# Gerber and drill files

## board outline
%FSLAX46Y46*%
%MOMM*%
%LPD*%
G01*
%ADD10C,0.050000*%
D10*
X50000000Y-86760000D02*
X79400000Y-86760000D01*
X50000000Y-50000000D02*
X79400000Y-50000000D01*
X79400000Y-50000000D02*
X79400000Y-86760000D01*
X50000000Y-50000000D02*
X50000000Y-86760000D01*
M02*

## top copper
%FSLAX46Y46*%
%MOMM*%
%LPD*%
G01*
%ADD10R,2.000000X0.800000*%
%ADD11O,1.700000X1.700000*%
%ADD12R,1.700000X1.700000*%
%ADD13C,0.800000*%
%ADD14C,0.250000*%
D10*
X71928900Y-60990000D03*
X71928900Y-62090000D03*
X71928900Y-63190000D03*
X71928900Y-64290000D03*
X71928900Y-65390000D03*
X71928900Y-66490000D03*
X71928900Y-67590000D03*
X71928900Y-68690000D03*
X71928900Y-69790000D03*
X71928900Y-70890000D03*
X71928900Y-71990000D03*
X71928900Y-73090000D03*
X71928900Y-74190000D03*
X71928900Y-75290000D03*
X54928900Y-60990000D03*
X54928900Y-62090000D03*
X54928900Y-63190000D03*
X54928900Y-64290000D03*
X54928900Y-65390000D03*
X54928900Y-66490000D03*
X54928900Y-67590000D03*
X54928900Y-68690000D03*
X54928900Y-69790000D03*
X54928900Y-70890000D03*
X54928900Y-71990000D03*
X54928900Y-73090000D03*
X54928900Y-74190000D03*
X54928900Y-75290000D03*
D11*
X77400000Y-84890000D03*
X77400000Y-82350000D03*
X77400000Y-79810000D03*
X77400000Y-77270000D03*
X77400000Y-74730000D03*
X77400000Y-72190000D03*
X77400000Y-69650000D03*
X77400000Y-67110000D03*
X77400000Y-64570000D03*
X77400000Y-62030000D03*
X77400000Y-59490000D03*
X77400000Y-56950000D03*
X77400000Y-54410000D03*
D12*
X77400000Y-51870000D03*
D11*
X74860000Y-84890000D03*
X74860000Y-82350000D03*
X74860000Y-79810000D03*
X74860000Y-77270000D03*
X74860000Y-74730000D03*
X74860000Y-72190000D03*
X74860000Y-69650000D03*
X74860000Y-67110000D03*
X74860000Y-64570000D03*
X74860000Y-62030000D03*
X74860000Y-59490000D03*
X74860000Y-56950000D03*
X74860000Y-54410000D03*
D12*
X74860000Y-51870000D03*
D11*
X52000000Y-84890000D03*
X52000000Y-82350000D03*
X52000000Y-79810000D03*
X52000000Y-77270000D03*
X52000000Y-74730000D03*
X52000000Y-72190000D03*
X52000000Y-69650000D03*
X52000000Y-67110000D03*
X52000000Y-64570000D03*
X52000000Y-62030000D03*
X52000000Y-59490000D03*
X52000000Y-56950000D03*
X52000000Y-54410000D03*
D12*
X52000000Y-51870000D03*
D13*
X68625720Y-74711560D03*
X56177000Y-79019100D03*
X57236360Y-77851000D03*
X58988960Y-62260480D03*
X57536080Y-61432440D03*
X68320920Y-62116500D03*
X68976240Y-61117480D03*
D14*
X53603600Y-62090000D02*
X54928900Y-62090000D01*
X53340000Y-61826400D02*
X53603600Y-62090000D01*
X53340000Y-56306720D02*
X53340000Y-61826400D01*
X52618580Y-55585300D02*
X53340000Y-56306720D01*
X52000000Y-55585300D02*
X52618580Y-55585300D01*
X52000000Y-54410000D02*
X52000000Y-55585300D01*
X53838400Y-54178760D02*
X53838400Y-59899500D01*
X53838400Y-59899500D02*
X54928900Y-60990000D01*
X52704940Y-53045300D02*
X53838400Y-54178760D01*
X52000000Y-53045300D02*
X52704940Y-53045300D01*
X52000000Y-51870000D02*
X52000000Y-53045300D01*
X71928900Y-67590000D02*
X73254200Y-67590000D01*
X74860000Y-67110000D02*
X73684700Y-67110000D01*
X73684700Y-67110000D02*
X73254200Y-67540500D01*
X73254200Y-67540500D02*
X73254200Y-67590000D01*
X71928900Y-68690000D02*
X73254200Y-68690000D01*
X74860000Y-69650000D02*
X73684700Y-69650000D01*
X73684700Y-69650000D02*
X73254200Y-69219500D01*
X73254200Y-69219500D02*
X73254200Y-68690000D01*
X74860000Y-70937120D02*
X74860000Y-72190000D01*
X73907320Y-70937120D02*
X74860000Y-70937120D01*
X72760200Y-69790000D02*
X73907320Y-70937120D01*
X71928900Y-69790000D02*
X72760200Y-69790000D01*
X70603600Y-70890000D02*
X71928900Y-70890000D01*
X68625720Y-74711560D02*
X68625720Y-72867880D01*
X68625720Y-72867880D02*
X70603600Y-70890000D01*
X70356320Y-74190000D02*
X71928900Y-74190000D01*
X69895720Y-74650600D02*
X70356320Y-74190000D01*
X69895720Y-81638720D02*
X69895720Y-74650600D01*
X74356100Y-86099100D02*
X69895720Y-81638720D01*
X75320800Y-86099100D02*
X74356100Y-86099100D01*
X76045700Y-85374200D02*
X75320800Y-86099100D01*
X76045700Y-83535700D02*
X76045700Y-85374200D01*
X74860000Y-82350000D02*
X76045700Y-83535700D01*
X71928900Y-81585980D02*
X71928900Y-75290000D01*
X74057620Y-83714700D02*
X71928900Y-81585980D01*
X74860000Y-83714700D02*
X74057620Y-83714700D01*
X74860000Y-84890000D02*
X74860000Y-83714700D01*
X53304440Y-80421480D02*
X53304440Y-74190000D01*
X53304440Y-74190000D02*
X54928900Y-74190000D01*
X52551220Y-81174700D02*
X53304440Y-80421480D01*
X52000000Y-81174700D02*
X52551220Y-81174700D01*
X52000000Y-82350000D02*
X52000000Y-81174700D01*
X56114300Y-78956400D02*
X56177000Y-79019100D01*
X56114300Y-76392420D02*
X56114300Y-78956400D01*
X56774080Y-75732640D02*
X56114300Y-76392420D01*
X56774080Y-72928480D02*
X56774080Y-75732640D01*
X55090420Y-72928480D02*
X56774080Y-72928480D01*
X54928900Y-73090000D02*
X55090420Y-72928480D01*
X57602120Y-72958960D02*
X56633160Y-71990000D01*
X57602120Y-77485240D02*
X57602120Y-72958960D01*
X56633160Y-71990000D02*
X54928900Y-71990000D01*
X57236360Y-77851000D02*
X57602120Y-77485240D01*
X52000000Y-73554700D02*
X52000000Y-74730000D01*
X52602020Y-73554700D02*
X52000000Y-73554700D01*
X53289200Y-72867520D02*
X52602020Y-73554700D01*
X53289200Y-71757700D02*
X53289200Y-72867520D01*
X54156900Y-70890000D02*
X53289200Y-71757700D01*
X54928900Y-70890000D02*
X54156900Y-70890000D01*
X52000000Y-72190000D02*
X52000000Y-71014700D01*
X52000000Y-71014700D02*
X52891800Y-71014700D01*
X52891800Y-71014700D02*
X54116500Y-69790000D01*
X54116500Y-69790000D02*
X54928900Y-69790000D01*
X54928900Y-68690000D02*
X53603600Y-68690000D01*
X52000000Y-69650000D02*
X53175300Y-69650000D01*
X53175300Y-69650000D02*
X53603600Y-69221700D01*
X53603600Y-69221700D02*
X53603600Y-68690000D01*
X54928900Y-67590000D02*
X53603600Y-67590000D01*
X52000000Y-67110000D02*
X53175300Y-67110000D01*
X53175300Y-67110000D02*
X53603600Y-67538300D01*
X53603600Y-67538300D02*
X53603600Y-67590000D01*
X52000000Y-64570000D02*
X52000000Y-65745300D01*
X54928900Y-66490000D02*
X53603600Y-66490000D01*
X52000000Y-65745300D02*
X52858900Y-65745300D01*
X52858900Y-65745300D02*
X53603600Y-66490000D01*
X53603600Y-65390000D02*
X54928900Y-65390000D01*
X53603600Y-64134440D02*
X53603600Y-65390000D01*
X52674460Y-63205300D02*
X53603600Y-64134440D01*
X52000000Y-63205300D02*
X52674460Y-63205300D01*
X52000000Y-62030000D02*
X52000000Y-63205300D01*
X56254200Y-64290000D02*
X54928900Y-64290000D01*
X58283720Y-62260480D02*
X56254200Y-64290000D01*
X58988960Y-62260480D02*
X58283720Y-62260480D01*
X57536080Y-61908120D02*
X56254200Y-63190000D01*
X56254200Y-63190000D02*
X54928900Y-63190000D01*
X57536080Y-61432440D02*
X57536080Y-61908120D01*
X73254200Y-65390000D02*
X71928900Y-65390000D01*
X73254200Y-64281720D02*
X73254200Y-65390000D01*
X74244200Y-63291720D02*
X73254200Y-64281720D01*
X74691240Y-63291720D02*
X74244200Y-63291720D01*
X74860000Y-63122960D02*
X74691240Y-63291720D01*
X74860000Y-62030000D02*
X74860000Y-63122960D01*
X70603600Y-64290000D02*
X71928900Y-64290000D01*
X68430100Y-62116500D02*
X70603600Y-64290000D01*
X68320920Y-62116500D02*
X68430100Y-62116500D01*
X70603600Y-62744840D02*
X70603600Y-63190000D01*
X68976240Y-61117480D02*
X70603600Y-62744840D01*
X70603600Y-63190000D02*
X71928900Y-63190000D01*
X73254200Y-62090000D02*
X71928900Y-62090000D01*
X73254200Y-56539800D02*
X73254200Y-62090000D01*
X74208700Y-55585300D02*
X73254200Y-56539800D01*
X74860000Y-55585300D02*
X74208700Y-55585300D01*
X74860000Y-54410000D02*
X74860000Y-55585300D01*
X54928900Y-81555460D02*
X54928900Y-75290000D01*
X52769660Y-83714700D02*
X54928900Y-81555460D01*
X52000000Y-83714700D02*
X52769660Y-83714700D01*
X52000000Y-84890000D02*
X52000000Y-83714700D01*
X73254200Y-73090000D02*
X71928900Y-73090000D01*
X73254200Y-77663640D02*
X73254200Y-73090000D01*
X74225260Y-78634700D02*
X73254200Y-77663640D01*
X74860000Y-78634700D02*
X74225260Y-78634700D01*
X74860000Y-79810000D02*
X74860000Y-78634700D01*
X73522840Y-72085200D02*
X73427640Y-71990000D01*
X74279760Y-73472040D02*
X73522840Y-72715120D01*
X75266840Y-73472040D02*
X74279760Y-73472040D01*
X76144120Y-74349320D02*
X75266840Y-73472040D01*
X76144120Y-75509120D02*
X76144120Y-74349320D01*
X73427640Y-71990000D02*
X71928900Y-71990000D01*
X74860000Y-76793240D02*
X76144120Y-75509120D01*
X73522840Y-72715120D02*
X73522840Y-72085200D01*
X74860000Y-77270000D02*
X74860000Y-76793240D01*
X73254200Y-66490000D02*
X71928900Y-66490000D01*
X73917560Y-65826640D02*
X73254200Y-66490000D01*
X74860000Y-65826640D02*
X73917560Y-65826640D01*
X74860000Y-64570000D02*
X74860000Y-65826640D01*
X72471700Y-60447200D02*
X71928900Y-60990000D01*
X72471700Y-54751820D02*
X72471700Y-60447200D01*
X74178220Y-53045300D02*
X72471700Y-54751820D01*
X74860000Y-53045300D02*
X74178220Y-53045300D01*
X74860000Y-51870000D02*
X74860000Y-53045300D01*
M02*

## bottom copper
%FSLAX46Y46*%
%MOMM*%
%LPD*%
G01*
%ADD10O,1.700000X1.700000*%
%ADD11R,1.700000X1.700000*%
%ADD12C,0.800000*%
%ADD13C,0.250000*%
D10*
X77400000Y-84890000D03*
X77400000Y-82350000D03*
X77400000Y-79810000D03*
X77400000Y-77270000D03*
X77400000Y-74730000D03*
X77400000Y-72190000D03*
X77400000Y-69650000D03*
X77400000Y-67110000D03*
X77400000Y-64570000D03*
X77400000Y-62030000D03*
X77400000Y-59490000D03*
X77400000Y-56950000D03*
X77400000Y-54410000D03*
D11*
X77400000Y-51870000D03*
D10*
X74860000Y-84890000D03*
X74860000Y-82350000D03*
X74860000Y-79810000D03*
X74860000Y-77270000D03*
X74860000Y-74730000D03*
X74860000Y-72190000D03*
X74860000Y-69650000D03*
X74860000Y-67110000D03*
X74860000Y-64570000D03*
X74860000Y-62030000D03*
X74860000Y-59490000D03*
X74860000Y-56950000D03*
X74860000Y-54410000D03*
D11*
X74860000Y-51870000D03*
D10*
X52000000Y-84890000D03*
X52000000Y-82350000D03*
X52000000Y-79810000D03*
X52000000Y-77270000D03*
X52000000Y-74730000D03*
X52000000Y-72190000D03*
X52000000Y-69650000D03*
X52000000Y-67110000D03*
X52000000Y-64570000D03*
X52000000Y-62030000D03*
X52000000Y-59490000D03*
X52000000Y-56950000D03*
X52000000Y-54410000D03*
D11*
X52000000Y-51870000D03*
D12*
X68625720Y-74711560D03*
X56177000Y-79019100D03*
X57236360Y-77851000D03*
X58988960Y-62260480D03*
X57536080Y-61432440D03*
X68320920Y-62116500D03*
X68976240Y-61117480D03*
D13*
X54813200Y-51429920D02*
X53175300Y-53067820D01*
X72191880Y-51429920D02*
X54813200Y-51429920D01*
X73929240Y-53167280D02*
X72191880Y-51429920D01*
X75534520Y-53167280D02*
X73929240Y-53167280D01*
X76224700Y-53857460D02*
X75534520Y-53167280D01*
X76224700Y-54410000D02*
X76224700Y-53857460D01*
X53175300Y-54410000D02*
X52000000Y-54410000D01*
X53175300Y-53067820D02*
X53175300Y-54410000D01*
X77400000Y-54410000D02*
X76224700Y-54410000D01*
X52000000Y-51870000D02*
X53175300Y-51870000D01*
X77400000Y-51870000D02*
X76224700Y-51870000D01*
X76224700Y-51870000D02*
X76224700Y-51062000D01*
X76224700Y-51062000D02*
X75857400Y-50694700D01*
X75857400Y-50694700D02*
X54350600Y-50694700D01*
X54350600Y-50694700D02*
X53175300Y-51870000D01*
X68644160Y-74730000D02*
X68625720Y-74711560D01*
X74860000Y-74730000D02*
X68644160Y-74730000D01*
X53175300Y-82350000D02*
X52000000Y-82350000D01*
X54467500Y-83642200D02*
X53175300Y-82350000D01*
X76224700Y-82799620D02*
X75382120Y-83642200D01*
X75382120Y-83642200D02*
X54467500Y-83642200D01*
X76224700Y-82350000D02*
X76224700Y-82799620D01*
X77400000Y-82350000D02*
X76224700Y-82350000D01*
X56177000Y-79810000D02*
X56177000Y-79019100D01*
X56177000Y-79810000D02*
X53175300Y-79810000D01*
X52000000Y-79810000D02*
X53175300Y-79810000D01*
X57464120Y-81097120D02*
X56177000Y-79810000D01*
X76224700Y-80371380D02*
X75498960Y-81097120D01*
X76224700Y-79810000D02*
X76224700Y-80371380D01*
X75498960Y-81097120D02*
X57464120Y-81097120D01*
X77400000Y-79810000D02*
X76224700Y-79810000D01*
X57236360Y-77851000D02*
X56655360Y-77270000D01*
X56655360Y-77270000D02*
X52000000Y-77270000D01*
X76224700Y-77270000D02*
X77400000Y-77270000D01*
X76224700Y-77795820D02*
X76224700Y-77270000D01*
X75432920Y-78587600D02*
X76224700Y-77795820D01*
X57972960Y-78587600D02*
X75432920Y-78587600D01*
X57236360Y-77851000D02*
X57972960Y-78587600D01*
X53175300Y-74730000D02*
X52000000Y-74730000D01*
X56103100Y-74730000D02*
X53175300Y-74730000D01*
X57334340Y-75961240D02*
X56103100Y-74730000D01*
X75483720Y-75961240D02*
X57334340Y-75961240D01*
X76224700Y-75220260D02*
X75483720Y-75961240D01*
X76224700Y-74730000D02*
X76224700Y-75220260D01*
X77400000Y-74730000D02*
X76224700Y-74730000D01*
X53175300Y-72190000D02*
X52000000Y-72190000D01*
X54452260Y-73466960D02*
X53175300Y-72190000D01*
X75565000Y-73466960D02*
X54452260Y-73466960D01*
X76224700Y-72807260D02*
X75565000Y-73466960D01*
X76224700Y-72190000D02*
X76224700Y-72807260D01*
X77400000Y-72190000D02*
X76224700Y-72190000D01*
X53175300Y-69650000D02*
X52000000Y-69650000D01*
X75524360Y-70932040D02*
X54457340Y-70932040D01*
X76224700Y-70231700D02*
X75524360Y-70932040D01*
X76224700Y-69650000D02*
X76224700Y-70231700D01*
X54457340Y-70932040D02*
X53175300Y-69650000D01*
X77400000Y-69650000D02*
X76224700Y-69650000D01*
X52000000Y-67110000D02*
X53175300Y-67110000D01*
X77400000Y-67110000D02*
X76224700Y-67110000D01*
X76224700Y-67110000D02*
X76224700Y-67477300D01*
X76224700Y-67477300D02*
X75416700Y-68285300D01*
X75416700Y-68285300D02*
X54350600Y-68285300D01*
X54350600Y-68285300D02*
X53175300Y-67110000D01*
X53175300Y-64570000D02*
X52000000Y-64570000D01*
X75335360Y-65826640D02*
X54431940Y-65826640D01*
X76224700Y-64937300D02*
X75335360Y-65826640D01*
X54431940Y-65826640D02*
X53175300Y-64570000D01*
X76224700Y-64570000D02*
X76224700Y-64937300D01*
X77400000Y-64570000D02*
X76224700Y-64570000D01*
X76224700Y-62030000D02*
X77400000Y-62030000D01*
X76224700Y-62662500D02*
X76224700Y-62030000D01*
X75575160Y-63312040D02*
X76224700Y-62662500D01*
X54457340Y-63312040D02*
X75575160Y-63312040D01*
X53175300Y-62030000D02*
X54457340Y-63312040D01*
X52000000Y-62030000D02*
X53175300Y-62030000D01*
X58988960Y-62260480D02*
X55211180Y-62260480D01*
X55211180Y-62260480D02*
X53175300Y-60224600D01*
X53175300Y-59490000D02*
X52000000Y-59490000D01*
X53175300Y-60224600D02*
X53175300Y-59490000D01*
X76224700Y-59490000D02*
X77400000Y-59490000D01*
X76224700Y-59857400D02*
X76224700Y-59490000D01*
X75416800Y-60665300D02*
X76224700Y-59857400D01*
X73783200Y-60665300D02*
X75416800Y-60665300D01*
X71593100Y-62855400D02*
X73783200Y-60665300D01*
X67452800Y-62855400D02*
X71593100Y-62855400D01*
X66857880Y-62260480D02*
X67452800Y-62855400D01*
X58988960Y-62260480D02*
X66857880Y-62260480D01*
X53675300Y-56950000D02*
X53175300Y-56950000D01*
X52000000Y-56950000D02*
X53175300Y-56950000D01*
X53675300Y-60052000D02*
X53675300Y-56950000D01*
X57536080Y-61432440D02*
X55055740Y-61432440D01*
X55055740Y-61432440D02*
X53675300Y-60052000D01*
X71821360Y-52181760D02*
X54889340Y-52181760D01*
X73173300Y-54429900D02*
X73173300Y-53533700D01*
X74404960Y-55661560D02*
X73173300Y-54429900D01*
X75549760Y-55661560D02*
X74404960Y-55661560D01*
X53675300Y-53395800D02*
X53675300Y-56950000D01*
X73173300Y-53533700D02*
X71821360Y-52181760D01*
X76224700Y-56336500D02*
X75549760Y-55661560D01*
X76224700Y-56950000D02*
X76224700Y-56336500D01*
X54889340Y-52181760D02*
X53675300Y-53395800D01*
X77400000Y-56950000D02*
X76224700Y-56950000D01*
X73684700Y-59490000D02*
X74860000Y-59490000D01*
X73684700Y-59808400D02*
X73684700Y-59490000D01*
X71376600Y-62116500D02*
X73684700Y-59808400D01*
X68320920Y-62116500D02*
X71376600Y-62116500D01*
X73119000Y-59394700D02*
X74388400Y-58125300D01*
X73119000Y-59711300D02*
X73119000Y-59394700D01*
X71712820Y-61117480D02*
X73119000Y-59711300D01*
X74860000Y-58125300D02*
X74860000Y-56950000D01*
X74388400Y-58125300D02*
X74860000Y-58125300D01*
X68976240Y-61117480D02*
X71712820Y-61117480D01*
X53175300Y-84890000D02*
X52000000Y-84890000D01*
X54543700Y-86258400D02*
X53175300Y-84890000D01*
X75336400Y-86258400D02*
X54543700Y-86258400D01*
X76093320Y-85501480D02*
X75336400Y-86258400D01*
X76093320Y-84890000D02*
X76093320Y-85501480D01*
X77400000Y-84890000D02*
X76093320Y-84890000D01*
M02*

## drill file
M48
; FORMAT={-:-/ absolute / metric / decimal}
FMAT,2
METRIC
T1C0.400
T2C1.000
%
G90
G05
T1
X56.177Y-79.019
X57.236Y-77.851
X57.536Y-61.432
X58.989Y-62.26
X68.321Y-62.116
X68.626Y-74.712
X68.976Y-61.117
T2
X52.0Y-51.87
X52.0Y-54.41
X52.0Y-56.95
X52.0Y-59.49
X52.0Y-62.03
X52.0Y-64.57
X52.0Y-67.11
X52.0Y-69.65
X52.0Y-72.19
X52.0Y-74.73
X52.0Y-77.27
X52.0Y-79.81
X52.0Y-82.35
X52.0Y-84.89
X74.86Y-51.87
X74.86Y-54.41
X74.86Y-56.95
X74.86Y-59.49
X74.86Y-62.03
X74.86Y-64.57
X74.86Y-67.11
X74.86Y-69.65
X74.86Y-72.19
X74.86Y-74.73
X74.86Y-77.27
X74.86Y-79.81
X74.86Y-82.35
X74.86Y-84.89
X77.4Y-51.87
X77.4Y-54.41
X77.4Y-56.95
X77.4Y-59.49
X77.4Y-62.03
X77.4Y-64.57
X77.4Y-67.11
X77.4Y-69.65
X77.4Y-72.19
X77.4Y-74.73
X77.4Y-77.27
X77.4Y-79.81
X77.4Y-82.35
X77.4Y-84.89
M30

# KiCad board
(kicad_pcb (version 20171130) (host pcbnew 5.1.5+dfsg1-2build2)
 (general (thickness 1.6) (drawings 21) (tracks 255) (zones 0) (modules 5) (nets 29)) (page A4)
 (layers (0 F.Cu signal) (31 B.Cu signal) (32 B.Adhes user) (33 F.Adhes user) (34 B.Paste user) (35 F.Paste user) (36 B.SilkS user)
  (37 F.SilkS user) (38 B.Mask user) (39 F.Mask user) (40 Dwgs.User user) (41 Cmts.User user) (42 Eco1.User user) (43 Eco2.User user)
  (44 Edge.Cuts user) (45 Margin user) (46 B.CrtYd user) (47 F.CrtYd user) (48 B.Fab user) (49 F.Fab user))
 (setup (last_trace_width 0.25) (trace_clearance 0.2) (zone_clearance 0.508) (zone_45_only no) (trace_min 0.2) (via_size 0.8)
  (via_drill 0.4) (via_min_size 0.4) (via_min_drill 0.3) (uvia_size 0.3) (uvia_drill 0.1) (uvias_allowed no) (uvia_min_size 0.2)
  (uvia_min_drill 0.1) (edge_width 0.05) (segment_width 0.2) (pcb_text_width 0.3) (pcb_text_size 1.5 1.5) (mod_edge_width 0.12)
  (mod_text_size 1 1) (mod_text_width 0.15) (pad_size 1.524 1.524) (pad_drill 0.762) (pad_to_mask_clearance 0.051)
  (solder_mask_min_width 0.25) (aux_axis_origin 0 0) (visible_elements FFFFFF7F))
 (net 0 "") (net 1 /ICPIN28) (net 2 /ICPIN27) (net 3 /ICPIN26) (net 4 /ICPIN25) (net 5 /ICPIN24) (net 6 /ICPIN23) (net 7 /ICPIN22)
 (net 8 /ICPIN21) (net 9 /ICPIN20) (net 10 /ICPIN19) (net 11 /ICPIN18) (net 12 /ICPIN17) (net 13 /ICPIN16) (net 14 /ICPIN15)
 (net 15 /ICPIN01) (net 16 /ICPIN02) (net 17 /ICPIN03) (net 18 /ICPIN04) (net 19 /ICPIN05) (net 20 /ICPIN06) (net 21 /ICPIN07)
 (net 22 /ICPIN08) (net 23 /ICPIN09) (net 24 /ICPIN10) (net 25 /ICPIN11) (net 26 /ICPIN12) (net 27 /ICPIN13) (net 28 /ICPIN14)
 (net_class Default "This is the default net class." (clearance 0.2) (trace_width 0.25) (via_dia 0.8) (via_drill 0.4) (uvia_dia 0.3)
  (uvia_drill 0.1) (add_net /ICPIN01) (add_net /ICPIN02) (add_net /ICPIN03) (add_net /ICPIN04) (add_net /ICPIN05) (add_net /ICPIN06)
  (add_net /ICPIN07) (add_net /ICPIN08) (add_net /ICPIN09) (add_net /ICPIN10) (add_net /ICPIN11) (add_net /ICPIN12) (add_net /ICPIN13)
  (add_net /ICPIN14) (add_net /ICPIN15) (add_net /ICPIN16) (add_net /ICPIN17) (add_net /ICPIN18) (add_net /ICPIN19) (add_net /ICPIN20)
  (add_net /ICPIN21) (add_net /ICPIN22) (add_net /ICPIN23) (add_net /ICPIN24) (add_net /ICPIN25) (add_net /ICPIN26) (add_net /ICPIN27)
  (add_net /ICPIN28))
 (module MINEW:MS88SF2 (layer F.Cu) (at 63.4289 65)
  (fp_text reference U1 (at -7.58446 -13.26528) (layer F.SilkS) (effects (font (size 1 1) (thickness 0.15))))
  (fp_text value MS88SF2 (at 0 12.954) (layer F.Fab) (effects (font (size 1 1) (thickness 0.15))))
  (pad 28 smd rect (at 8.5 -4.01) (size 2 0.8) (layers F.Cu F.Paste F.Mask) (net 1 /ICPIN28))
  (pad 27 smd rect (at 8.5 -2.91) (size 2 0.8) (layers F.Cu F.Paste F.Mask) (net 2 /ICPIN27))
  (pad 26 smd rect (at 8.5 -1.81) (size 2 0.8) (layers F.Cu F.Paste F.Mask) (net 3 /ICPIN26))
  (pad 25 smd rect (at 8.5 -0.71) (size 2 0.8) (layers F.Cu F.Paste F.Mask) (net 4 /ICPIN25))
  (pad 24 smd rect (at 8.5 0.39) (size 2 0.8) (layers F.Cu F.Paste F.Mask) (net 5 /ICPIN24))
  (pad 23 smd rect (at 8.5 1.49) (size 2 0.8) (layers F.Cu F.Paste F.Mask) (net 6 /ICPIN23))
  (pad 22 smd rect (at 8.5 2.59) (size 2 0.8) (layers F.Cu F.Paste F.Mask) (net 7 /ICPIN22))
  (pad 21 smd rect (at 8.5 3.69) (size 2 0.8) (layers F.Cu F.Paste F.Mask) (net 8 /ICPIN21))
  (pad 20 smd rect (at 8.5 4.79) (size 2 0.8) (layers F.Cu F.Paste F.Mask) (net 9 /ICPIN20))
  (pad 19 smd rect (at 8.5 5.89) (size 2 0.8) (layers F.Cu F.Paste F.Mask) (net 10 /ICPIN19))
  (pad 18 smd rect (at 8.5 6.99) (size 2 0.8) (layers F.Cu F.Paste F.Mask) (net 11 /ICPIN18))
  (pad 17 smd rect (at 8.5 8.09) (size 2 0.8) (layers F.Cu F.Paste F.Mask) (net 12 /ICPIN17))
  (pad 16 smd rect (at 8.5 9.19) (size 2 0.8) (layers F.Cu F.Paste F.Mask) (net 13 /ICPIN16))
  (pad 15 smd rect (at 8.5 10.29) (size 2 0.8) (layers F.Cu F.Paste F.Mask) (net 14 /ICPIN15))
  (pad 1 smd rect (at -8.5 -4.01) (size 2 0.8) (layers F.Cu F.Paste F.Mask) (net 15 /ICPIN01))
  (pad 2 smd rect (at -8.5 -2.91) (size 2 0.8) (layers F.Cu F.Paste F.Mask) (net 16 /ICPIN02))
  (pad 3 smd rect (at -8.5 -1.81) (size 2 0.8) (layers F.Cu F.Paste F.Mask) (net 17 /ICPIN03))
  (pad 4 smd rect (at -8.5 -0.71) (size 2 0.8) (layers F.Cu F.Paste F.Mask) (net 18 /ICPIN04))
  (pad 5 smd rect (at -8.5 0.39) (size 2 0.8) (layers F.Cu F.Paste F.Mask) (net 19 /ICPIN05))
  (pad 6 smd rect (at -8.5 1.49) (size 2 0.8) (layers F.Cu F.Paste F.Mask) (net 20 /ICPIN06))
  (pad 7 smd rect (at -8.5 2.59) (size 2 0.8) (layers F.Cu F.Paste F.Mask) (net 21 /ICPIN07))
  (pad 8 smd rect (at -8.5 3.69) (size 2 0.8) (layers F.Cu F.Paste F.Mask) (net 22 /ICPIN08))
  (pad 9 smd rect (at -8.5 4.79) (size 2 0.8) (layers F.Cu F.Paste F.Mask) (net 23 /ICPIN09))
  (pad 10 smd rect (at -8.5 5.89) (size 2 0.8) (layers F.Cu F.Paste F.Mask) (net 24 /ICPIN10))
  (pad 11 smd rect (at -8.5 6.99) (size 2 0.8) (layers F.Cu F.Paste F.Mask) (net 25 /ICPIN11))
  (pad 12 smd rect (at -8.5 8.09) (size 2 0.8) (layers F.Cu F.Paste F.Mask) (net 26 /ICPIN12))
  (pad 13 smd rect (at -8.5 9.19) (size 2 0.8) (layers F.Cu F.Paste F.Mask) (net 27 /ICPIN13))
  (pad 14 smd rect (at -8.5 10.29) (size 2 0.8) (layers F.Cu F.Paste F.Mask) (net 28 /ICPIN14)))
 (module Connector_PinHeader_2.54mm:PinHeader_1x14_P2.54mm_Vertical (layer F.Cu) (at 77.4 51.87)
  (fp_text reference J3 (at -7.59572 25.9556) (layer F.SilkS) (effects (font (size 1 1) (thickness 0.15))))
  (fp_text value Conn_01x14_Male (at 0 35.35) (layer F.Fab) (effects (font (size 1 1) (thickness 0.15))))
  (pad 14 thru_hole oval (at 0 33.02) (size 1.7 1.7) (drill 1) (layers *.Cu *.Mask) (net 28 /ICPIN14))
  (pad 13 thru_hole oval (at 0 30.48) (size 1.7 1.7) (drill 1) (layers *.Cu *.Mask) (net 27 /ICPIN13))
  (pad 12 thru_hole oval (at 0 27.94) (size 1.7 1.7) (drill 1) (layers *.Cu *.Mask) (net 26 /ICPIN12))
  (pad 11 thru_hole oval (at 0 25.4) (size 1.7 1.7) (drill 1) (layers *.Cu *.Mask) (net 25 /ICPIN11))
  (pad 10 thru_hole oval (at 0 22.86) (size 1.7 1.7) (drill 1) (layers *.Cu *.Mask) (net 24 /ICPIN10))
  (pad 9 thru_hole oval (at 0 20.32) (size 1.7 1.7) (drill 1) (layers *.Cu *.Mask) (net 23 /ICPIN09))
  (pad 8 thru_hole oval (at 0 17.78) (size 1.7 1.7) (drill 1) (layers *.Cu *.Mask) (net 22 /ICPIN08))
  (pad 7 thru_hole oval (at 0 15.24) (size 1.7 1.7) (drill 1) (layers *.Cu *.Mask) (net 21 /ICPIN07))
  (pad 6 thru_hole oval (at 0 12.7) (size 1.7 1.7) (drill 1) (layers *.Cu *.Mask) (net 20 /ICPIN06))
  (pad 5 thru_hole oval (at 0 10.16) (size 1.7 1.7) (drill 1) (layers *.Cu *.Mask) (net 19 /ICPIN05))
  (pad 4 thru_hole oval (at 0 7.62) (size 1.7 1.7) (drill 1) (layers *.Cu *.Mask) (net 18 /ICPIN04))
  (pad 3 thru_hole oval (at 0 5.08) (size 1.7 1.7) (drill 1) (layers *.Cu *.Mask) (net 17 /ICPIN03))
  (pad 2 thru_hole oval (at 0 2.54) (size 1.7 1.7) (drill 1) (layers *.Cu *.Mask) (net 16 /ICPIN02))
  (pad 1 thru_hole rect (at 0 0) (size 1.7 1.7) (drill 1) (layers *.Cu *.Mask) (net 15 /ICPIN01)))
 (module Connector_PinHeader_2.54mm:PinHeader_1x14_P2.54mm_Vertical (layer F.Cu) (at 74.86 51.87)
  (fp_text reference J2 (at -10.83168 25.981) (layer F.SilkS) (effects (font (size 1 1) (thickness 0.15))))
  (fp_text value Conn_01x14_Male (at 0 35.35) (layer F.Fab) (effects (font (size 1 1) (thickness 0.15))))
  (pad 14 thru_hole oval (at 0 33.02) (size 1.7 1.7) (drill 1) (layers *.Cu *.Mask) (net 14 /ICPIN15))
  (pad 13 thru_hole oval (at 0 30.48) (size 1.7 1.7) (drill 1) (layers *.Cu *.Mask) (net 13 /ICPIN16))
  (pad 12 thru_hole oval (at 0 27.94) (size 1.7 1.7) (drill 1) (layers *.Cu *.Mask) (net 12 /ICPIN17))
  (pad 11 thru_hole oval (at 0 25.4) (size 1.7 1.7) (drill 1) (layers *.Cu *.Mask) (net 11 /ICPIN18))
  (pad 10 thru_hole oval (at 0 22.86) (size 1.7 1.7) (drill 1) (layers *.Cu *.Mask) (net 10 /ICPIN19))
  (pad 9 thru_hole oval (at 0 20.32) (size 1.7 1.7) (drill 1) (layers *.Cu *.Mask) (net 9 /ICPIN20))
  (pad 8 thru_hole oval (at 0 17.78) (size 1.7 1.7) (drill 1) (layers *.Cu *.Mask) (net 8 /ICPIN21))
  (pad 7 thru_hole oval (at 0 15.24) (size 1.7 1.7) (drill 1) (layers *.Cu *.Mask) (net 7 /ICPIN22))
  (pad 6 thru_hole oval (at 0 12.7) (size 1.7 1.7) (drill 1) (layers *.Cu *.Mask) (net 6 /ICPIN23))
  (pad 5 thru_hole oval (at 0 10.16) (size 1.7 1.7) (drill 1) (layers *.Cu *.Mask) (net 5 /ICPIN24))
  (pad 4 thru_hole oval (at 0 7.62) (size 1.7 1.7) (drill 1) (layers *.Cu *.Mask) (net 4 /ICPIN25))
  (pad 3 thru_hole oval (at 0 5.08) (size 1.7 1.7) (drill 1) (layers *.Cu *.Mask) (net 3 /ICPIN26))
  (pad 2 thru_hole oval (at 0 2.54) (size 1.7 1.7) (drill 1) (layers *.Cu *.Mask) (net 2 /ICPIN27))
  (pad 1 thru_hole rect (at 0 0) (size 1.7 1.7) (drill 1) (layers *.Cu *.Mask) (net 1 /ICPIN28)))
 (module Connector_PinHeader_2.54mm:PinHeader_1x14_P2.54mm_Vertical (layer F.Cu) (at 52 51.87)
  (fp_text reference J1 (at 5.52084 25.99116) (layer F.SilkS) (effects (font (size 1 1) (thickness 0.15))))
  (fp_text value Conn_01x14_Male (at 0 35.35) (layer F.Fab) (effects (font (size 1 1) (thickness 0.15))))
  (pad 14 thru_hole oval (at 0 33.02) (size 1.7 1.7) (drill 1) (layers *.Cu *.Mask) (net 28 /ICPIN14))
  (pad 13 thru_hole oval (at 0 30.48) (size 1.7 1.7) (drill 1) (layers *.Cu *.Mask) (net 27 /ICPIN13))
  (pad 12 thru_hole oval (at 0 27.94) (size 1.7 1.7) (drill 1) (layers *.Cu *.Mask) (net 26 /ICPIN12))
  (pad 11 thru_hole oval (at 0 25.4) (size 1.7 1.7) (drill 1) (layers *.Cu *.Mask) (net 25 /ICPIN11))
  (pad 10 thru_hole oval (at 0 22.86) (size 1.7 1.7) (drill 1) (layers *.Cu *.Mask) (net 24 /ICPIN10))
  (pad 9 thru_hole oval (at 0 20.32) (size 1.7 1.7) (drill 1) (layers *.Cu *.Mask) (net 23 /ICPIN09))
  (pad 8 thru_hole oval (at 0 17.78) (size 1.7 1.7) (drill 1) (layers *.Cu *.Mask) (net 22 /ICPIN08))
  (pad 7 thru_hole oval (at 0 15.24) (size 1.7 1.7) (drill 1) (layers *.Cu *.Mask) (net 21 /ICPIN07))
  (pad 6 thru_hole oval (at 0 12.7) (size 1.7 1.7) (drill 1) (layers *.Cu *.Mask) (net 20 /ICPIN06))
  (pad 5 thru_hole oval (at 0 10.16) (size 1.7 1.7) (drill 1) (layers *.Cu *.Mask) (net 19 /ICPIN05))
  (pad 4 thru_hole oval (at 0 7.62) (size 1.7 1.7) (drill 1) (layers *.Cu *.Mask) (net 18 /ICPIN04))
  (pad 3 thru_hole oval (at 0 5.08) (size 1.7 1.7) (drill 1) (layers *.Cu *.Mask) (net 17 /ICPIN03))
  (pad 2 thru_hole oval (at 0 2.54) (size 1.7 1.7) (drill 1) (layers *.Cu *.Mask) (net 16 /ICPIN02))
  (pad 1 thru_hole rect (at 0 0) (size 1.7 1.7) (drill 1) (layers *.Cu *.Mask) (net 15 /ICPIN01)))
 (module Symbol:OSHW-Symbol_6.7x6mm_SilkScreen (layer F.Cu) (at 63.2714 56.68264)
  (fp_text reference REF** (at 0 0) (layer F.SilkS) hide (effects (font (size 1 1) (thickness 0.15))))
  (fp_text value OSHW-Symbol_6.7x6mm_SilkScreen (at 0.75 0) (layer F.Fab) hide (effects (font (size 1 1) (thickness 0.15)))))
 (gr_line (start 50 86.76) (end 79.4 86.76) (layer Edge.Cuts) (width 0.05))
 (gr_line (start 50 50) (end 79.4 50) (layer Edge.Cuts) (width 0.05))
 (gr_line (start 79.4 50) (end 79.4 86.76) (layer Edge.Cuts) (width 0.05))
 (gr_line (start 50 50) (end 50 86.76) (layer Edge.Cuts) (width 0.05))
 (segment (start 54.8132 51.42992) (end 53.1753 53.06782) (width 0.25) (layer B.Cu) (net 16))
 (segment (start 72.19188 51.42992) (end 54.8132 51.42992) (width 0.25) (layer B.Cu) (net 16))
 (segment (start 73.92924 53.16728) (end 72.19188 51.42992) (width 0.25) (layer B.Cu) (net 16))
 (segment (start 75.53452 53.16728) (end 73.92924 53.16728) (width 0.25) (layer B.Cu) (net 16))
 (segment (start 76.2247 53.85746) (end 75.53452 53.16728) (width 0.25) (layer B.Cu) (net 16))
 (segment (start 76.2247 54.41) (end 76.2247 53.85746) (width 0.25) (layer B.Cu) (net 16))
 (segment (start 53.1753 54.41) (end 52 54.41) (width 0.25) (layer B.Cu) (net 16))
 (segment (start 53.1753 53.06782) (end 53.1753 54.41) (width 0.25) (layer B.Cu) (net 16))
 (segment (start 77.4 54.41) (end 76.2247 54.41) (width 0.25) (layer B.Cu) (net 16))
 (segment (start 53.6036 62.09) (end 54.9289 62.09) (width 0.25) (layer F.Cu) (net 16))
 (segment (start 53.34 61.8264) (end 53.6036 62.09) (width 0.25) (layer F.Cu) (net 16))
 (segment (start 53.34 56.30672) (end 53.34 61.8264) (width 0.25) (layer F.Cu) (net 16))
 (segment (start 52.61858 55.5853) (end 53.34 56.30672) (width 0.25) (layer F.Cu) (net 16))
 (segment (start 52 55.5853) (end 52.61858 55.5853) (width 0.25) (layer F.Cu) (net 16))
 (segment (start 52 54.41) (end 52 55.5853) (width 0.25) (layer F.Cu) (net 16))
 (segment (start 52 51.87) (end 53.1753 51.87) (width 0.25) (layer B.Cu) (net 15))
 (segment (start 77.4 51.87) (end 76.2247 51.87) (width 0.25) (layer B.Cu) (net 15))
 (segment (start 76.2247 51.87) (end 76.2247 51.062) (width 0.25) (layer B.Cu) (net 15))
 (segment (start 76.2247 51.062) (end 75.8574 50.6947) (width 0.25) (layer B.Cu) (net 15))
 (segment (start 75.8574 50.6947) (end 54.3506 50.6947) (width 0.25) (layer B.Cu) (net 15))
 (segment (start 54.3506 50.6947) (end 53.1753 51.87) (width 0.25) (layer B.Cu) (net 15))
 (segment (start 53.8384 54.17876) (end 53.8384 59.8995) (width 0.25) (layer F.Cu) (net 15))
 (segment (start 53.8384 59.8995) (end 54.9289 60.99) (width 0.25) (layer F.Cu) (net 15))
 (segment (start 52.70494 53.0453) (end 53.8384 54.17876) (width 0.25) (layer F.Cu) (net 15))
 (segment (start 52 53.0453) (end 52.70494 53.0453) (width 0.25) (layer F.Cu) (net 15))
 (segment (start 52 51.87) (end 52 53.0453) (width 0.25) (layer F.Cu) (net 15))
 (segment (start 71.9289 67.59) (end 73.2542 67.59) (width 0.25) (layer F.Cu) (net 7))
 (segment (start 74.86 67.11) (end 73.6847 67.11) (width 0.25) (layer F.Cu) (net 7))
 (segment (start 73.6847 67.11) (end 73.2542 67.5405) (width 0.25) (layer F.Cu) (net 7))
 (segment (start 73.2542 67.5405) (end 73.2542 67.59) (width 0.25) (layer F.Cu) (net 7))
 (segment (start 71.9289 68.69) (end 73.2542 68.69) (width 0.25) (layer F.Cu) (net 8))
 (segment (start 74.86 69.65) (end 73.6847 69.65) (width 0.25) (layer F.Cu) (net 8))
 (segment (start 73.6847 69.65) (end 73.2542 69.2195) (width 0.25) (layer F.Cu) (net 8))
 (segment (start 73.2542 69.2195) (end 73.2542 68.69) (width 0.25) (layer F.Cu) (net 8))
 (segment (start 74.86 70.93712) (end 74.86 72.19) (width 0.25) (layer F.Cu) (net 9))
 (segment (start 73.90732 70.93712) (end 74.86 70.93712) (width 0.25) (layer F.Cu) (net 9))
 (segment (start 72.7602 69.79) (end 73.90732 70.93712) (width 0.25) (layer F.Cu) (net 9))
 (segment (start 71.9289 69.79) (end 72.7602 69.79) (width 0.25) (layer F.Cu) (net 9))
 (segment (start 70.6036 70.89) (end 71.9289 70.89) (width 0.25) (layer F.Cu) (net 10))
 (segment (start 68.62572 74.71156) (end 68.62572 72.86788) (width 0.25) (layer F.Cu) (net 10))
 (segment (start 68.64416 74.73) (end 68.62572 74.71156) (width 0.25) (layer B.Cu) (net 10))
 (segment (start 68.62572 72.86788) (end 70.6036 70.89) (width 0.25) (layer F.Cu) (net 10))
 (segment (start 74.86 74.73) (end 68.64416 74.73) (width 0.25) (layer B.Cu) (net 10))
 (via (at 68.62572 74.71156) (size 0.8) (drill 0.4) (layers F.Cu B.Cu) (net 10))
 (segment (start 70.35632 74.19) (end 71.9289 74.19) (width 0.25) (layer F.Cu) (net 13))
 (segment (start 69.89572 74.6506) (end 70.35632 74.19) (width 0.25) (layer F.Cu) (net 13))
 (segment (start 69.89572 81.63872) (end 69.89572 74.6506) (width 0.25) (layer F.Cu) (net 13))
 (segment (start 74.3561 86.0991) (end 69.89572 81.63872) (width 0.25) (layer F.Cu) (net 13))
 (segment (start 75.3208 86.0991) (end 74.3561 86.0991) (width 0.25) (layer F.Cu) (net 13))
 (segment (start 76.0457 85.3742) (end 75.3208 86.0991) (width 0.25) (layer F.Cu) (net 13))
 (segment (start 76.0457 83.5357) (end 76.0457 85.3742) (width 0.25) (layer F.Cu) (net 13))
 (segment (start 74.86 82.35) (end 76.0457 83.5357) (width 0.25) (layer F.Cu) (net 13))
 (segment (start 71.9289 81.58598) (end 71.9289 75.29) (width 0.25) (layer F.Cu) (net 14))
 (segment (start 74.05762 83.7147) (end 71.9289 81.58598) (width 0.25) (layer F.Cu) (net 14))
 (segment (start 74.86 83.7147) (end 74.05762 83.7147) (width 0.25) (layer F.Cu) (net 14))
 (segment (start 74.86 84.89) (end 74.86 83.7147) (width 0.25) (layer F.Cu) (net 14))
 (segment (start 53.1753 82.35) (end 52 82.35) (width 0.25) (layer B.Cu) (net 27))
 (segment (start 54.4675 83.6422) (end 53.1753 82.35) (width 0.25) (layer B.Cu) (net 27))
 (segment (start 76.2247 82.79962) (end 75.38212 83.6422) (width 0.25) (layer B.Cu) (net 27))
 (segment (start 75.38212 83.6422) (end 54.4675 83.6422) (width 0.25) (layer B.Cu) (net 27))
 (segment (start 76.2247 82.35) (end 76.2247 82.79962) (width 0.25) (layer B.Cu) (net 27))
 (segment (start 77.4 82.35) (end 76.2247 82.35) (width 0.25) (layer B.Cu) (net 27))
 (segment (start 53.30444 80.42148) (end 53.30444 74.19) (width 0.25) (layer F.Cu) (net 27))
 (segment (start 53.30444 74.19) (end 54.9289 74.19) (width 0.25) (layer F.Cu) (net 27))
 (segment (start 52.55122 81.1747) (end 53.30444 80.42148) (width 0.25) (layer F.Cu) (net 27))
 (segment (start 52 81.1747) (end 52.55122 81.1747) (width 0.25) (layer F.Cu) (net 27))
 (segment (start 52 82.35) (end 52 81.1747) (width 0.25) (layer F.Cu) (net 27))
 (segment (start 56.177 79.81) (end 56.177 79.0191) (width 0.25) (layer B.Cu) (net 26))
 (segment (start 56.177 79.81) (end 53.1753 79.81) (width 0.25) (layer B.Cu) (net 26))
 (segment (start 52 79.81) (end 53.1753 79.81) (width 0.25) (layer B.Cu) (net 26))
 (via (at 56.177 79.0191) (size 0.8) (layers F.Cu B.Cu) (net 26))
 (segment (start 56.1143 78.9564) (end 56.177 79.0191) (width 0.25) (layer F.Cu) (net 26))
 (segment (start 56.1143 76.39242) (end 56.1143 78.9564) (width 0.25) (layer F.Cu) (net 26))
 (segment (start 56.77408 75.73264) (end 56.1143 76.39242) (width 0.25) (layer F.Cu) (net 26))
 (segment (start 56.77408 72.92848) (end 56.77408 75.73264) (width 0.25) (layer F.Cu) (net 26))
 (segment (start 55.09042 72.92848) (end 56.77408 72.92848) (width 0.25) (layer F.Cu) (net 26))
 (segment (start 54.9289 73.09) (end 55.09042 72.92848) (width 0.25) (layer F.Cu) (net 26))
 (segment (start 57.46412 81.09712) (end 56.177 79.81) (width 0.25) (layer B.Cu) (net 26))
 (segment (start 76.2247 80.37138) (end 75.49896 81.09712) (width 0.25) (layer B.Cu) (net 26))
 (segment (start 76.2247 79.81) (end 76.2247 80.37138) (width 0.25) (layer B.Cu) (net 26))
 (segment (start 75.49896 81.09712) (end 57.46412 81.09712) (width 0.25) (layer B.Cu) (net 26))
 (segment (start 77.4 79.81) (end 76.2247 79.81) (width 0.25) (layer B.Cu) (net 26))
 (segment (start 57.23636 77.851) (end 56.65536 77.27) (width 0.25) (layer B.Cu) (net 25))
 (segment (start 56.65536 77.27) (end 52 77.27) (width 0.25) (layer B.Cu) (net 25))
 (via (at 57.23636 77.851) (size 0.8) (drill 0.4) (layers F.Cu B.Cu) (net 25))
 (segment (start 57.60212 72.95896) (end 56.63316 71.99) (width 0.25) (layer F.Cu) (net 25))
 (segment (start 57.60212 77.48524) (end 57.60212 72.95896) (width 0.25) (layer F.Cu) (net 25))
 (segment (start 56.63316 71.99) (end 54.9289 71.99) (width 0.25) (layer F.Cu) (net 25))
 (segment (start 57.23636 77.851) (end 57.60212 77.48524) (width 0.25) (layer F.Cu) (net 25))
 (segment (start 76.2247 77.27) (end 77.4 77.27) (width 0.25) (layer B.Cu) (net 25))
 (segment (start 76.2247 77.79582) (end 76.2247 77.27) (width 0.25) (layer B.Cu) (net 25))
 (segment (start 75.43292 78.5876) (end 76.2247 77.79582) (width 0.25) (layer B.Cu) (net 25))
 (segment (start 57.97296 78.5876) (end 75.43292 78.5876) (width 0.25) (layer B.Cu) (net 25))
 (segment (start 57.23636 77.851) (end 57.97296 78.5876) (width 0.25) (layer B.Cu) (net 25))
 (segment (start 53.1753 74.73) (end 52 74.73) (width 0.25) (layer B.Cu) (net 24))
 (segment (start 56.1031 74.73) (end 53.1753 74.73) (width 0.25) (layer B.Cu) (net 24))
 (segment (start 57.33434 75.96124) (end 56.1031 74.73) (width 0.25) (layer B.Cu) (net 24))
 (segment (start 75.48372 75.96124) (end 57.33434 75.96124) (width 0.25) (layer B.Cu) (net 24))
 (segment (start 76.2247 75.22026) (end 75.48372 75.96124) (width 0.25) (layer B.Cu) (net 24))
 (segment (start 76.2247 74.73) (end 76.2247 75.22026) (width 0.25) (layer B.Cu) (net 24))
 (segment (start 77.4 74.73) (end 76.2247 74.73) (width 0.25) (layer B.Cu) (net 24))
 (segment (start 52 73.5547) (end 52 74.73) (width 0.25) (layer F.Cu) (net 24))
 (segment (start 52.60202 73.5547) (end 52 73.5547) (width 0.25) (layer F.Cu) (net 24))
 (segment (start 53.2892 72.86752) (end 52.60202 73.5547) (width 0.25) (layer F.Cu) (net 24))
 (segment (start 53.2892 71.7577) (end 53.2892 72.86752) (width 0.25) (layer F.Cu) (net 24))
 (segment (start 54.1569 70.89) (end 53.2892 71.7577) (width 0.25) (layer F.Cu) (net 24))
 (segment (start 54.9289 70.89) (end 54.1569 70.89) (width 0.25) (layer F.Cu) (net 24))
 (segment (start 52 72.19) (end 52 71.0147) (width 0.25) (layer F.Cu) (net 23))
 (segment (start 52 71.0147) (end 52.8918 71.0147) (width 0.25) (layer F.Cu) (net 23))
 (segment (start 52.8918 71.0147) (end 54.1165 69.79) (width 0.25) (layer F.Cu) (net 23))
 (segment (start 54.1165 69.79) (end 54.9289 69.79) (width 0.25) (layer F.Cu) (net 23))
 (segment (start 53.1753 72.19) (end 52 72.19) (width 0.25) (layer B.Cu) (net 23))
 (segment (start 54.45226 73.46696) (end 53.1753 72.19) (width 0.25) (layer B.Cu) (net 23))
 (segment (start 75.565 73.46696) (end 54.45226 73.46696) (width 0.25) (layer B.Cu) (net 23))
 (segment (start 76.2247 72.80726) (end 75.565 73.46696) (width 0.25) (layer B.Cu) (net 23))
 (segment (start 76.2247 72.19) (end 76.2247 72.80726) (width 0.25) (layer B.Cu) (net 23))
 (segment (start 77.4 72.19) (end 76.2247 72.19) (width 0.25) (layer B.Cu) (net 23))
 (segment (start 54.9289 68.69) (end 53.6036 68.69) (width 0.25) (layer F.Cu) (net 22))
 (segment (start 52 69.65) (end 53.1753 69.65) (width 0.25) (layer F.Cu) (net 22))
 (segment (start 53.1753 69.65) (end 53.6036 69.2217) (width 0.25) (layer F.Cu) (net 22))
 (segment (start 53.6036 69.2217) (end 53.6036 68.69) (width 0.25) (layer F.Cu) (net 22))
 (segment (start 53.1753 69.65) (end 52 69.65) (width 0.25) (layer B.Cu) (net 22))
 (segment (start 75.52436 70.93204) (end 54.45734 70.93204) (width 0.25) (layer B.Cu) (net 22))
 (segment (start 76.2247 70.2317) (end 75.52436 70.93204) (width 0.25) (layer B.Cu) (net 22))
 (segment (start 76.2247 69.65) (end 76.2247 70.2317) (width 0.25) (layer B.Cu) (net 22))
 (segment (start 54.45734 70.93204) (end 53.1753 69.65) (width 0.25) (layer B.Cu) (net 22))
 (segment (start 77.4 69.65) (end 76.2247 69.65) (width 0.25) (layer B.Cu) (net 22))
 (segment (start 52 67.11) (end 53.1753 67.11) (width 0.25) (layer B.Cu) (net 21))
 (segment (start 77.4 67.11) (end 76.2247 67.11) (width 0.25) (layer B.Cu) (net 21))
 (segment (start 76.2247 67.11) (end 76.2247 67.4773) (width 0.25) (layer B.Cu) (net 21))
 (segment (start 76.2247 67.4773) (end 75.4167 68.2853) (width 0.25) (layer B.Cu) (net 21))
 (segment (start 75.4167 68.2853) (end 54.3506 68.2853) (width 0.25) (layer B.Cu) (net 21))
 (segment (start 54.3506 68.2853) (end 53.1753 67.11) (width 0.25) (layer B.Cu) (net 21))
 (segment (start 54.9289 67.59) (end 53.6036 67.59) (width 0.25) (layer F.Cu) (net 21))
 (segment (start 52 67.11) (end 53.1753 67.11) (width 0.25) (layer F.Cu) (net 21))
 (segment (start 53.1753 67.11) (end 53.6036 67.5383) (width 0.25) (layer F.Cu) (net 21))
 (segment (start 53.6036 67.5383) (end 53.6036 67.59) (width 0.25) (layer F.Cu) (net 21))
 (segment (start 52 64.57) (end 52 65.7453) (width 0.25) (layer F.Cu) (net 20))
 (segment (start 54.9289 66.49) (end 53.6036 66.49) (width 0.25) (layer F.Cu) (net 20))
 (segment (start 52 65.7453) (end 52.8589 65.7453) (width 0.25) (layer F.Cu) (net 20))
 (segment (start 52.8589 65.7453) (end 53.6036 66.49) (width 0.25) (layer F.Cu) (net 20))
 (segment (start 53.1753 64.57) (end 52 64.57) (width 0.25) (layer B.Cu) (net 20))
 (segment (start 75.33536 65.82664) (end 54.43194 65.82664) (width 0.25) (layer B.Cu) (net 20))
 (segment (start 76.2247 64.9373) (end 75.33536 65.82664) (width 0.25) (layer B.Cu) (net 20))
 (segment (start 54.43194 65.82664) (end 53.1753 64.57) (width 0.25) (layer B.Cu) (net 20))
 (segment (start 76.2247 64.57) (end 76.2247 64.9373) (width 0.25) (layer B.Cu) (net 20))
 (segment (start 77.4 64.57) (end 76.2247 64.57) (width 0.25) (layer B.Cu) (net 20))
 (segment (start 53.6036 65.39) (end 54.9289 65.39) (width 0.25) (layer F.Cu) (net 19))
 (segment (start 53.6036 64.13444) (end 53.6036 65.39) (width 0.25) (layer F.Cu) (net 19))
 (segment (start 52.67446 63.2053) (end 53.6036 64.13444) (width 0.25) (layer F.Cu) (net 19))
 (segment (start 52 63.2053) (end 52.67446 63.2053) (width 0.25) (layer F.Cu) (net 19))
 (segment (start 52 62.03) (end 52 63.2053) (width 0.25) (layer F.Cu) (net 19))
 (segment (start 76.2247 62.03) (end 77.4 62.03) (width 0.25) (layer B.Cu) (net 19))
 (segment (start 76.2247 62.6625) (end 76.2247 62.03) (width 0.25) (layer B.Cu) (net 19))
 (segment (start 75.57516 63.31204) (end 76.2247 62.6625) (width 0.25) (layer B.Cu) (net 19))
 (segment (start 54.45734 63.31204) (end 75.57516 63.31204) (width 0.25) (layer B.Cu) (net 19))
 (segment (start 53.1753 62.03) (end 54.45734 63.31204) (width 0.25) (layer B.Cu) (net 19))
 (segment (start 52 62.03) (end 53.1753 62.03) (width 0.25) (layer B.Cu) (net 19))
 (segment (start 56.2542 64.29) (end 54.9289 64.29) (width 0.25) (layer F.Cu) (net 18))
 (via (at 58.98896 62.26048) (size 0.8) (drill 0.4) (layers F.Cu B.Cu) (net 18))
 (segment (start 58.98896 62.26048) (end 55.21118 62.26048) (width 0.25) (layer B.Cu) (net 18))
 (segment (start 55.21118 62.26048) (end 53.1753 60.2246) (width 0.25) (layer B.Cu) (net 18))
 (segment (start 58.28372 62.26048) (end 56.2542 64.29) (width 0.25) (layer F.Cu) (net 18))
 (segment (start 53.1753 59.49) (end 52 59.49) (width 0.25) (layer B.Cu) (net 18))
 (segment (start 53.1753 60.2246) (end 53.1753 59.49) (width 0.25) (layer B.Cu) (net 18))
 (segment (start 58.98896 62.26048) (end 58.28372 62.26048) (width 0.25) (layer F.Cu) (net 18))
 (segment (start 76.2247 59.49) (end 77.4 59.49) (width 0.25) (layer B.Cu) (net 18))
 (segment (start 76.2247 59.8574) (end 76.2247 59.49) (width 0.25) (layer B.Cu) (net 18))
 (segment (start 75.4168 60.6653) (end 76.2247 59.8574) (width 0.25) (layer B.Cu) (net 18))
 (segment (start 73.7832 60.6653) (end 75.4168 60.6653) (width 0.25) (layer B.Cu) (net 18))
 (segment (start 71.5931 62.8554) (end 73.7832 60.6653) (width 0.25) (layer B.Cu) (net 18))
 (segment (start 67.4528 62.8554) (end 71.5931 62.8554) (width 0.25) (layer B.Cu) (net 18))
 (segment (start 66.85788 62.26048) (end 67.4528 62.8554) (width 0.25) (layer B.Cu) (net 18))
 (segment (start 58.98896 62.26048) (end 66.85788 62.26048) (width 0.25) (layer B.Cu) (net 18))
 (segment (start 53.6753 56.95) (end 53.1753 56.95) (width 0.25) (layer B.Cu) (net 17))
 (segment (start 52 56.95) (end 53.1753 56.95) (width 0.25) (layer B.Cu) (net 17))
 (segment (start 53.6753 60.052) (end 53.6753 56.95) (width 0.25) (layer B.Cu) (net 17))
 (segment (start 57.53608 61.43244) (end 55.05574 61.43244) (width 0.25) (layer B.Cu) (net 17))
 (segment (start 55.05574 61.43244) (end 53.6753 60.052) (width 0.25) (layer B.Cu) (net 17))
 (segment (start 57.53608 61.90812) (end 56.2542 63.19) (width 0.25) (layer F.Cu) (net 17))
 (segment (start 56.2542 63.19) (end 54.9289 63.19) (width 0.25) (layer F.Cu) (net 17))
 (segment (start 57.53608 61.43244) (end 57.53608 61.90812) (width 0.25) (layer F.Cu) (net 17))
 (via (at 57.53608 61.43244) (size 0.8) (drill 0.4) (layers F.Cu B.Cu) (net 17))
 (segment (start 71.82136 52.18176) (end 54.88934 52.18176) (width 0.25) (layer B.Cu) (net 17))
 (segment (start 73.1733 54.4299) (end 73.1733 53.5337) (width 0.25) (layer B.Cu) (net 17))
 (segment (start 74.40496 55.66156) (end 73.1733 54.4299) (width 0.25) (layer B.Cu) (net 17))
 (segment (start 75.54976 55.66156) (end 74.40496 55.66156) (width 0.25) (layer B.Cu) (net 17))
 (segment (start 53.6753 53.3958) (end 53.6753 56.95) (width 0.25) (layer B.Cu) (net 17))
 (segment (start 73.1733 53.5337) (end 71.82136 52.18176) (width 0.25) (layer B.Cu) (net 17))
 (segment (start 76.2247 56.3365) (end 75.54976 55.66156) (width 0.25) (layer B.Cu) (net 17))
 (segment (start 76.2247 56.95) (end 76.2247 56.3365) (width 0.25) (layer B.Cu) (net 17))
 (segment (start 54.88934 52.18176) (end 53.6753 53.3958) (width 0.25) (layer B.Cu) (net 17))
 (segment (start 77.4 56.95) (end 76.2247 56.95) (width 0.25) (layer B.Cu) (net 17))
 (segment (start 73.2542 65.39) (end 71.9289 65.39) (width 0.25) (layer F.Cu) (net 5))
 (segment (start 73.2542 64.28172) (end 73.2542 65.39) (width 0.25) (layer F.Cu) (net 5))
 (segment (start 74.2442 63.29172) (end 73.2542 64.28172) (width 0.25) (layer F.Cu) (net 5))
 (segment (start 74.69124 63.29172) (end 74.2442 63.29172) (width 0.25) (layer F.Cu) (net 5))
 (segment (start 74.86 63.12296) (end 74.69124 63.29172) (width 0.25) (layer F.Cu) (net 5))
 (segment (start 74.86 62.03) (end 74.86 63.12296) (width 0.25) (layer F.Cu) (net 5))
 (segment (start 70.6036 64.29) (end 71.9289 64.29) (width 0.25) (layer F.Cu) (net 4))
 (segment (start 68.4301 62.1165) (end 70.6036 64.29) (width 0.25) (layer F.Cu) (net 4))
 (segment (start 73.6847 59.49) (end 74.86 59.49) (width 0.25) (layer B.Cu) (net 4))
 (segment (start 73.6847 59.8084) (end 73.6847 59.49) (width 0.25) (layer B.Cu) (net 4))
 (segment (start 71.3766 62.1165) (end 73.6847 59.8084) (width 0.25) (layer B.Cu) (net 4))
 (segment (start 68.32092 62.1165) (end 71.3766 62.1165) (width 0.25) (layer B.Cu) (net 4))
 (segment (start 68.32092 62.1165) (end 68.4301 62.1165) (width 0.25) (layer F.Cu) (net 4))
 (via (at 68.32092 62.1165) (size 0.8) (drill 0.4) (layers F.Cu B.Cu) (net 4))
 (segment (start 70.6036 62.74484) (end 70.6036 63.19) (width 0.25) (layer F.Cu) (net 3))
 (segment (start 68.97624 61.11748) (end 70.6036 62.74484) (width 0.25) (layer F.Cu) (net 3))
 (segment (start 70.6036 63.19) (end 71.9289 63.19) (width 0.25) (layer F.Cu) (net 3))
 (segment (start 73.119 59.3947) (end 74.3884 58.1253) (width 0.25) (layer B.Cu) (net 3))
 (segment (start 73.119 59.7113) (end 73.119 59.3947) (width 0.25) (layer B.Cu) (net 3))
 (segment (start 71.71282 61.11748) (end 73.119 59.7113) (width 0.25) (layer B.Cu) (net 3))
 (segment (start 74.86 58.1253) (end 74.86 56.95) (width 0.25) (layer B.Cu) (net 3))
 (segment (start 74.3884 58.1253) (end 74.86 58.1253) (width 0.25) (layer B.Cu) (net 3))
 (segment (start 68.97624 61.11748) (end 71.71282 61.11748) (width 0.25) (layer B.Cu) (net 3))
 (via (at 68.97624 61.11748) (size 0.8) (drill 0.4) (layers F.Cu B.Cu) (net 3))
 (segment (start 73.2542 62.09) (end 71.9289 62.09) (width 0.25) (layer F.Cu) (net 2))
 (segment (start 73.2542 56.5398) (end 73.2542 62.09) (width 0.25) (layer F.Cu) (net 2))
 (segment (start 74.2087 55.5853) (end 73.2542 56.5398) (width 0.25) (layer F.Cu) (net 2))
 (segment (start 74.86 55.5853) (end 74.2087 55.5853) (width 0.25) (layer F.Cu) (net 2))
 (segment (start 74.86 54.41) (end 74.86 55.5853) (width 0.25) (layer F.Cu) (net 2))
 (segment (start 53.1753 84.89) (end 52 84.89) (width 0.25) (layer B.Cu) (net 28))
 (segment (start 54.5437 86.2584) (end 53.1753 84.89) (width 0.25) (layer B.Cu) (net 28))
 (segment (start 75.3364 86.2584) (end 54.5437 86.2584) (width 0.25) (layer B.Cu) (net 28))
 (segment (start 76.09332 85.50148) (end 75.3364 86.2584) (width 0.25) (layer B.Cu) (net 28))
 (segment (start 76.09332 84.89) (end 76.09332 85.50148) (width 0.25) (layer B.Cu) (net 28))
 (segment (start 77.4 84.89) (end 76.09332 84.89) (width 0.25) (layer B.Cu) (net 28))
 (segment (start 54.9289 81.55546) (end 54.9289 75.29) (width 0.25) (layer F.Cu) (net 28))
 (segment (start 52.76966 83.7147) (end 54.9289 81.55546) (width 0.25) (layer F.Cu) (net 28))
 (segment (start 52 83.7147) (end 52.76966 83.7147) (width 0.25) (layer F.Cu) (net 28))
 (segment (start 52 84.89) (end 52 83.7147) (width 0.25) (layer F.Cu) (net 28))
 (segment (start 73.2542 73.09) (end 71.9289 73.09) (width 0.25) (layer F.Cu) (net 12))
 (segment (start 73.2542 77.66364) (end 73.2542 73.09) (width 0.25) (layer F.Cu) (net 12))
 (segment (start 74.22526 78.6347) (end 73.2542 77.66364) (width 0.25) (layer F.Cu) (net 12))
 (segment (start 74.86 78.6347) (end 74.22526 78.6347) (width 0.25) (layer F.Cu) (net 12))
 (segment (start 74.86 79.81) (end 74.86 78.6347) (width 0.25) (layer F.Cu) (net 12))
 (segment (start 73.52284 72.0852) (end 73.42764 71.99) (width 0.25) (layer F.Cu) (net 11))
 (segment (start 74.27976 73.47204) (end 73.52284 72.71512) (width 0.25) (layer F.Cu) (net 11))
 (segment (start 75.26684 73.47204) (end 74.27976 73.47204) (width 0.25) (layer F.Cu) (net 11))
 (segment (start 76.14412 74.34932) (end 75.26684 73.47204) (width 0.25) (layer F.Cu) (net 11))
 (segment (start 76.14412 75.50912) (end 76.14412 74.34932) (width 0.25) (layer F.Cu) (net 11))
 (segment (start 73.42764 71.99) (end 71.9289 71.99) (width 0.25) (layer F.Cu) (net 11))
 (segment (start 74.86 76.79324) (end 76.14412 75.50912) (width 0.25) (layer F.Cu) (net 11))
 (segment (start 73.52284 72.71512) (end 73.52284 72.0852) (width 0.25) (layer F.Cu) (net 11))
 (segment (start 74.86 77.27) (end 74.86 76.79324) (width 0.25) (layer F.Cu) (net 11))
 (segment (start 73.2542 66.49) (end 71.9289 66.49) (width 0.25) (layer F.Cu) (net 6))
 (segment (start 73.91756 65.82664) (end 73.2542 66.49) (width 0.25) (layer F.Cu) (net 6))
 (segment (start 74.86 65.82664) (end 73.91756 65.82664) (width 0.25) (layer F.Cu) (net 6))
 (segment (start 74.86 64.57) (end 74.86 65.82664) (width 0.25) (layer F.Cu) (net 6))
 (segment (start 72.4717 60.4472) (end 71.9289 60.99) (width 0.25) (layer F.Cu) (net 1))
 (segment (start 72.4717 54.75182) (end 72.4717 60.4472) (width 0.25) (layer F.Cu) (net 1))
 (segment (start 74.17822 53.0453) (end 72.4717 54.75182) (width 0.25) (layer F.Cu) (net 1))
 (segment (start 74.86 53.0453) (end 74.17822 53.0453) (width 0.25) (layer F.Cu) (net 1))
 (segment (start 74.86 51.87) (end 74.86 53.0453) (width 0.25) (layer F.Cu) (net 1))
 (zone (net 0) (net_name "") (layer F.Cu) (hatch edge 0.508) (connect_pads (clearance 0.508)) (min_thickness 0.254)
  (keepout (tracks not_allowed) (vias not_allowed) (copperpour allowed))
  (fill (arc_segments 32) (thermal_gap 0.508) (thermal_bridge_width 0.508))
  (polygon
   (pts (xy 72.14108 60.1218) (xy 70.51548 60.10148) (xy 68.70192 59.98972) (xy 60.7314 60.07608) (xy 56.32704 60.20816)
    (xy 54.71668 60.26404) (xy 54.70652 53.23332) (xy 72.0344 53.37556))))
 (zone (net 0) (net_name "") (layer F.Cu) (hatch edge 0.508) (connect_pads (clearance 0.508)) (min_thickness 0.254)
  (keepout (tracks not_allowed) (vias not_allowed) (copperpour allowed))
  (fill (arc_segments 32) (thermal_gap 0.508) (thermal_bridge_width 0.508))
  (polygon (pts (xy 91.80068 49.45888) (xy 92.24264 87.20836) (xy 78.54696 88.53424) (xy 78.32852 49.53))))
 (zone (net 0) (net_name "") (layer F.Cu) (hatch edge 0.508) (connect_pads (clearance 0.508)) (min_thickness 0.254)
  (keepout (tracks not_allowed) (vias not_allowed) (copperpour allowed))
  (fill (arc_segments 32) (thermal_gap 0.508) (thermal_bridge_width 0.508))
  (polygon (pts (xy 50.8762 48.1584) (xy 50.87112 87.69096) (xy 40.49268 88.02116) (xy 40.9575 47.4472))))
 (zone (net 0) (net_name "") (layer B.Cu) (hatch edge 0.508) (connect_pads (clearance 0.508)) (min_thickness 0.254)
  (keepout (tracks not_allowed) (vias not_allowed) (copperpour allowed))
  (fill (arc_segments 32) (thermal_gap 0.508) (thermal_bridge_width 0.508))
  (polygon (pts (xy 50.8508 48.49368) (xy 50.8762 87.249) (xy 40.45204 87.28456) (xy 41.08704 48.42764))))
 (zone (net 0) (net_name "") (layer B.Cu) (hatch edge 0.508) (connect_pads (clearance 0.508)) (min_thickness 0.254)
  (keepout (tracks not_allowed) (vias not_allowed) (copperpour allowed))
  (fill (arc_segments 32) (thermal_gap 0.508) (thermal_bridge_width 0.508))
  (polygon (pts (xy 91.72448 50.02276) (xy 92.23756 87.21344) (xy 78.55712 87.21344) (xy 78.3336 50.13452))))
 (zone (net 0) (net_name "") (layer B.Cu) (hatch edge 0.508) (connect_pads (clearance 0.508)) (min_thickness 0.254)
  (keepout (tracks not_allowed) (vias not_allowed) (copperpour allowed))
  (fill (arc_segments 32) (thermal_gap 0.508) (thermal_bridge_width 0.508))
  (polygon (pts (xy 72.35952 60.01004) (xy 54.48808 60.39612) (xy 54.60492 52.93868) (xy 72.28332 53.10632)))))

